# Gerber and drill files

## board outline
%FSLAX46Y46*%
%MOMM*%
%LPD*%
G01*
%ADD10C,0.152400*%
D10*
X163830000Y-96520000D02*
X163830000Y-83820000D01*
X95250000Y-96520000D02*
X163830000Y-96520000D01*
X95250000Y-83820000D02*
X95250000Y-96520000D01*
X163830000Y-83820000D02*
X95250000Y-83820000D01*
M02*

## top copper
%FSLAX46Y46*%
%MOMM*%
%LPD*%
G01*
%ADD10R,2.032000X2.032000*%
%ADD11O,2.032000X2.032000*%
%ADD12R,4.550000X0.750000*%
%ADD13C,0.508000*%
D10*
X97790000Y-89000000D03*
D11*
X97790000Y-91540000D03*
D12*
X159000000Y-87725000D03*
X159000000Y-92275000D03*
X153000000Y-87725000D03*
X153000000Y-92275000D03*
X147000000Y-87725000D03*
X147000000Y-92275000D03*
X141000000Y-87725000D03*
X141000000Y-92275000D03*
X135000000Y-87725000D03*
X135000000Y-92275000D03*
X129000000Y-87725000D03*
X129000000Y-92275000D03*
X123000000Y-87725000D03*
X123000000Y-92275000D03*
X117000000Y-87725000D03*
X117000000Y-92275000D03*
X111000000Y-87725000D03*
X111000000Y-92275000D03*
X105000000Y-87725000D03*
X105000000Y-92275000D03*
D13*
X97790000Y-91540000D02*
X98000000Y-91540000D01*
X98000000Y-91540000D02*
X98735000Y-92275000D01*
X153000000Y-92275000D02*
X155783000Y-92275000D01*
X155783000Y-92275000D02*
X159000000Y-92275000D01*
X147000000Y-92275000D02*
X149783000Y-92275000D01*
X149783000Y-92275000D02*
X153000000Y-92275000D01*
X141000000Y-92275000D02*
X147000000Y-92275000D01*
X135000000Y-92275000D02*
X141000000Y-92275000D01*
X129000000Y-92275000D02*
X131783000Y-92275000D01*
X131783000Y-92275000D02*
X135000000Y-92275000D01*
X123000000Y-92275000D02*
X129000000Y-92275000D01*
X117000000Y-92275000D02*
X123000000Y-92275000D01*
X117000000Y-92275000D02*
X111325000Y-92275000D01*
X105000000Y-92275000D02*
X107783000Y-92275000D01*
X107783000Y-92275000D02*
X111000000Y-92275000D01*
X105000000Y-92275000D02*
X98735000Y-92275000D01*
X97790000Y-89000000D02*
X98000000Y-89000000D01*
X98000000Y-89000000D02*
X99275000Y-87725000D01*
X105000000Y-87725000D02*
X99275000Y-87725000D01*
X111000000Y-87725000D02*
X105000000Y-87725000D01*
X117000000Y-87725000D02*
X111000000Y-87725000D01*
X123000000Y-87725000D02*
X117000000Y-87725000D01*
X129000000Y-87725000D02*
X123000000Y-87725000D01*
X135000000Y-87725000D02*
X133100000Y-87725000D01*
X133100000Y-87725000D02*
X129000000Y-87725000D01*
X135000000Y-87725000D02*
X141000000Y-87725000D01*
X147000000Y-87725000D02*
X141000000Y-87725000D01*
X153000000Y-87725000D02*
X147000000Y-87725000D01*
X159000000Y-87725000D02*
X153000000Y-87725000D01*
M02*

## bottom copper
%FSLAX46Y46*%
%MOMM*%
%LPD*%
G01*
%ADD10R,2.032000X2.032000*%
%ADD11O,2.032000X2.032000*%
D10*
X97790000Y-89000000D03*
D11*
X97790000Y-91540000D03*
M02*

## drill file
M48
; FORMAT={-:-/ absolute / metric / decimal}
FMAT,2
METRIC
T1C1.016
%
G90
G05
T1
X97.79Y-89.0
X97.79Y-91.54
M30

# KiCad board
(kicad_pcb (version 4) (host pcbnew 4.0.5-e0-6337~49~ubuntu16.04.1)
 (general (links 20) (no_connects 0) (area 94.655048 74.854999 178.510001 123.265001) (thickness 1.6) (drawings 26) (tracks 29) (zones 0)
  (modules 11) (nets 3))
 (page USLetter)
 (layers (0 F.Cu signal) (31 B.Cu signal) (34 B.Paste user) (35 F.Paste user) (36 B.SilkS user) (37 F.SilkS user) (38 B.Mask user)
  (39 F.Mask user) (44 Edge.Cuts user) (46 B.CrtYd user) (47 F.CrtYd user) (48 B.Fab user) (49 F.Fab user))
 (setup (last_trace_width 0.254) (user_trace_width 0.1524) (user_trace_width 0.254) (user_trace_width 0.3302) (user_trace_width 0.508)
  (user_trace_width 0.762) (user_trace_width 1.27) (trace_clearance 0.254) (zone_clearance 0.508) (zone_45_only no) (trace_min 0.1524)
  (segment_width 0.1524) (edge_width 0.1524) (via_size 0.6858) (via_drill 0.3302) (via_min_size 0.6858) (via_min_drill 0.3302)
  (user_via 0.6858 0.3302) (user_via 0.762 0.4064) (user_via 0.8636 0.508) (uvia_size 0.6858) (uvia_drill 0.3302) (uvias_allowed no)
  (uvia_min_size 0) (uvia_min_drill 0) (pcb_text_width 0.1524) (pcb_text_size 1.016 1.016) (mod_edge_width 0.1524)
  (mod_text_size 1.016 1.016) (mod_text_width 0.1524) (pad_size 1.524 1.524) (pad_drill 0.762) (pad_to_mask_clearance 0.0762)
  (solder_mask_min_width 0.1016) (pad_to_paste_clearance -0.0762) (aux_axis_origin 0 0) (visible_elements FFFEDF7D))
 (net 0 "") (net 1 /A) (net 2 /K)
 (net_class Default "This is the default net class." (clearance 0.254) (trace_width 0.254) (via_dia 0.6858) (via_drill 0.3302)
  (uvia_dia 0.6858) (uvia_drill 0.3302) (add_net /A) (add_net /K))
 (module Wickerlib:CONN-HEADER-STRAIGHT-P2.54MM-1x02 (layer F.Cu) (at 97.79 89)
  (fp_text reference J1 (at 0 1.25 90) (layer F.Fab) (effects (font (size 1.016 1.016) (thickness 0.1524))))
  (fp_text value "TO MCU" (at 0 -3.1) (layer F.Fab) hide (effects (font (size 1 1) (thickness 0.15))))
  (pad 1 thru_hole rect (at 0 0) (size 2.032 2.032) (drill 1.016) (layers *.Cu *.Mask F.SilkS) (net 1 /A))
  (pad 2 thru_hole oval (at 0 2.54) (size 2.032 2.032) (drill 1.016) (layers *.Cu *.Mask F.SilkS) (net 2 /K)))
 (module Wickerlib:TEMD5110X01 (layer F.Cu) (at 159 90)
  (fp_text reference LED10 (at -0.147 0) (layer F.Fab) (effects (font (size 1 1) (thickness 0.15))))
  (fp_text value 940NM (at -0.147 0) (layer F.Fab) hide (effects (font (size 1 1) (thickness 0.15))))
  (pad 2 smd rect (at 0 -2.275) (size 4.55 0.75) (layers F.Cu F.Paste F.Mask) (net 1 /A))
  (pad 1 smd rect (at 0 2.275) (size 4.55 0.75) (layers F.Cu F.Paste F.Mask) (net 2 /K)))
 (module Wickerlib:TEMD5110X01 (layer F.Cu) (at 153 90)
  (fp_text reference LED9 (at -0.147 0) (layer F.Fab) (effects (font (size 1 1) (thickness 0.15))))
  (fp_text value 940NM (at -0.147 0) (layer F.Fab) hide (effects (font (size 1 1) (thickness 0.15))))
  (pad 2 smd rect (at 0 -2.275) (size 4.55 0.75) (layers F.Cu F.Paste F.Mask) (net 1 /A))
  (pad 1 smd rect (at 0 2.275) (size 4.55 0.75) (layers F.Cu F.Paste F.Mask) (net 2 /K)))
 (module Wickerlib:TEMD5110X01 (layer F.Cu) (at 147 90)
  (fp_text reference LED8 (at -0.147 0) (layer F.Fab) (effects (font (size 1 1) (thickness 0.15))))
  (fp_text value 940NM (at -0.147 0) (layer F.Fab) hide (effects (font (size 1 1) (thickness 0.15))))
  (pad 2 smd rect (at 0 -2.275) (size 4.55 0.75) (layers F.Cu F.Paste F.Mask) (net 1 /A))
  (pad 1 smd rect (at 0 2.275) (size 4.55 0.75) (layers F.Cu F.Paste F.Mask) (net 2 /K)))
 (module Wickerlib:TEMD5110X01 (layer F.Cu) (at 141 90)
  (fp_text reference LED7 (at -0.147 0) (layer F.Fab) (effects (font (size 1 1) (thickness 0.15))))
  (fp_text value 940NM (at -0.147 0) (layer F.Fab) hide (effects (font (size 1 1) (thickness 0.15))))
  (pad 2 smd rect (at 0 -2.275) (size 4.55 0.75) (layers F.Cu F.Paste F.Mask) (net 1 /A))
  (pad 1 smd rect (at 0 2.275) (size 4.55 0.75) (layers F.Cu F.Paste F.Mask) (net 2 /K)))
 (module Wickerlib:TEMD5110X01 (layer F.Cu) (at 135 90)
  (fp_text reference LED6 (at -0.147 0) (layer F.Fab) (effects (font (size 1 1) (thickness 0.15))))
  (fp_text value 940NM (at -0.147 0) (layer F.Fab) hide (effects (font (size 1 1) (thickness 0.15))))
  (pad 2 smd rect (at 0 -2.275) (size 4.55 0.75) (layers F.Cu F.Paste F.Mask) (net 1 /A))
  (pad 1 smd rect (at 0 2.275) (size 4.55 0.75) (layers F.Cu F.Paste F.Mask) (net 2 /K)))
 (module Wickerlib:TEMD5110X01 (layer F.Cu) (at 129 90)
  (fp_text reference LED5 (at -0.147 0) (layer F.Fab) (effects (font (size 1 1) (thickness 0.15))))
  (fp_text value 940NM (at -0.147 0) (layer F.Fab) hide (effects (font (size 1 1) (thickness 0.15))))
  (pad 2 smd rect (at 0 -2.275) (size 4.55 0.75) (layers F.Cu F.Paste F.Mask) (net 1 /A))
  (pad 1 smd rect (at 0 2.275) (size 4.55 0.75) (layers F.Cu F.Paste F.Mask) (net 2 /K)))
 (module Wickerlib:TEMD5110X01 (layer F.Cu) (at 123 90)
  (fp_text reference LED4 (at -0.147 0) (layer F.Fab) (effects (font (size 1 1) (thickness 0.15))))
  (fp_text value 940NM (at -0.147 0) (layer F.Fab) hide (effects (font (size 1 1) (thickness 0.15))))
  (pad 2 smd rect (at 0 -2.275) (size 4.55 0.75) (layers F.Cu F.Paste F.Mask) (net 1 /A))
  (pad 1 smd rect (at 0 2.275) (size 4.55 0.75) (layers F.Cu F.Paste F.Mask) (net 2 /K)))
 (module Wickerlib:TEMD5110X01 (layer F.Cu) (at 117 90)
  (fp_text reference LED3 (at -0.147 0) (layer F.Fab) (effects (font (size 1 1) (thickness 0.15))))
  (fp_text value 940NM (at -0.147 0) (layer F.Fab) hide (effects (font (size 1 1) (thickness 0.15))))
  (pad 2 smd rect (at 0 -2.275) (size 4.55 0.75) (layers F.Cu F.Paste F.Mask) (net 1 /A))
  (pad 1 smd rect (at 0 2.275) (size 4.55 0.75) (layers F.Cu F.Paste F.Mask) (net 2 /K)))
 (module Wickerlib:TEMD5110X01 (layer F.Cu) (at 111 90)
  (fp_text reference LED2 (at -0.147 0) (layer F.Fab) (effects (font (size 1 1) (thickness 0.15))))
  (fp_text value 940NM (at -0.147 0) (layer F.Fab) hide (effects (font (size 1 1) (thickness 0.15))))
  (pad 2 smd rect (at 0 -2.275) (size 4.55 0.75) (layers F.Cu F.Paste F.Mask) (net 1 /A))
  (pad 1 smd rect (at 0 2.275) (size 4.55 0.75) (layers F.Cu F.Paste F.Mask) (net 2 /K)))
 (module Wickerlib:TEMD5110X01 (layer F.Cu) (at 105 90)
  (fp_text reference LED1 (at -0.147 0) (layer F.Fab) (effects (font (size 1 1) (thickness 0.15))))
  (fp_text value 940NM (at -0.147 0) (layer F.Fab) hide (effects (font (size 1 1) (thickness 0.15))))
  (pad 2 smd rect (at 0 -2.275) (size 4.55 0.75) (layers F.Cu F.Paste F.Mask) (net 1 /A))
  (pad 1 smd rect (at 0 2.275) (size 4.55 0.75) (layers F.Cu F.Paste F.Mask) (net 2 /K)))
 (gr_line (start 163.83 96.52) (end 163.83 83.82) (layer Edge.Cuts) (width 0.1524))
 (gr_line (start 95.25 96.52) (end 163.83 96.52) (layer Edge.Cuts) (width 0.1524))
 (gr_line (start 95.25 83.82) (end 95.25 96.52) (layer Edge.Cuts) (width 0.1524))
 (gr_line (start 163.83 83.82) (end 95.25 83.82) (layer Edge.Cuts) (width 0.1524))
 (segment (start 97.79 91.54) (end 98 91.54) (width 0.508) (layer F.Cu) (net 2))
 (segment (start 98 91.54) (end 98.735 92.275) (width 0.508) (layer F.Cu) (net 2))
 (segment (start 153 92.275) (end 155.783 92.275) (width 0.508) (layer F.Cu) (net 2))
 (segment (start 155.783 92.275) (end 159 92.275) (width 0.508) (layer F.Cu) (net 2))
 (segment (start 147 92.275) (end 149.783 92.275) (width 0.508) (layer F.Cu) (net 2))
 (segment (start 149.783 92.275) (end 153 92.275) (width 0.508) (layer F.Cu) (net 2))
 (segment (start 141 92.275) (end 147 92.275) (width 0.508) (layer F.Cu) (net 2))
 (segment (start 135 92.275) (end 141 92.275) (width 0.508) (layer F.Cu) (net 2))
 (segment (start 129 92.275) (end 131.783 92.275) (width 0.508) (layer F.Cu) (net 2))
 (segment (start 131.783 92.275) (end 135 92.275) (width 0.508) (layer F.Cu) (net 2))
 (segment (start 123 92.275) (end 129 92.275) (width 0.508) (layer F.Cu) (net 2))
 (segment (start 117 92.275) (end 123 92.275) (width 0.508) (layer F.Cu) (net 2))
 (segment (start 117 92.275) (end 111.325 92.275) (width 0.508) (layer F.Cu) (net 2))
 (segment (start 105 92.275) (end 107.783 92.275) (width 0.508) (layer F.Cu) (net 2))
 (segment (start 107.783 92.275) (end 111 92.275) (width 0.508) (layer F.Cu) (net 2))
 (segment (start 105 92.275) (end 98.735 92.275) (width 0.508) (layer F.Cu) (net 2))
 (segment (start 97.79 89) (end 98 89) (width 0.508) (layer F.Cu) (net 1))
 (segment (start 98 89) (end 99.275 87.725) (width 0.508) (layer F.Cu) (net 1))
 (segment (start 105 87.725) (end 99.275 87.725) (width 0.508) (layer F.Cu) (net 1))
 (segment (start 111 87.725) (end 105 87.725) (width 0.508) (layer F.Cu) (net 1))
 (segment (start 117 87.725) (end 111 87.725) (width 0.508) (layer F.Cu) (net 1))
 (segment (start 123 87.725) (end 117 87.725) (width 0.508) (layer F.Cu) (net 1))
 (segment (start 129 87.725) (end 123 87.725) (width 0.508) (layer F.Cu) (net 1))
 (segment (start 135 87.725) (end 133.1 87.725) (width 0.508) (layer F.Cu) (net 1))
 (segment (start 133.1 87.725) (end 129 87.725) (width 0.508) (layer F.Cu) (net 1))
 (segment (start 135 87.725) (end 141 87.725) (width 0.508) (layer F.Cu) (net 1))
 (segment (start 147 87.725) (end 141 87.725) (width 0.508) (layer F.Cu) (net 1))
 (segment (start 153 87.725) (end 147 87.725) (width 0.508) (layer F.Cu) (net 1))
 (segment (start 159 87.725) (end 153 87.725) (width 0.508) (layer F.Cu) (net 1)))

